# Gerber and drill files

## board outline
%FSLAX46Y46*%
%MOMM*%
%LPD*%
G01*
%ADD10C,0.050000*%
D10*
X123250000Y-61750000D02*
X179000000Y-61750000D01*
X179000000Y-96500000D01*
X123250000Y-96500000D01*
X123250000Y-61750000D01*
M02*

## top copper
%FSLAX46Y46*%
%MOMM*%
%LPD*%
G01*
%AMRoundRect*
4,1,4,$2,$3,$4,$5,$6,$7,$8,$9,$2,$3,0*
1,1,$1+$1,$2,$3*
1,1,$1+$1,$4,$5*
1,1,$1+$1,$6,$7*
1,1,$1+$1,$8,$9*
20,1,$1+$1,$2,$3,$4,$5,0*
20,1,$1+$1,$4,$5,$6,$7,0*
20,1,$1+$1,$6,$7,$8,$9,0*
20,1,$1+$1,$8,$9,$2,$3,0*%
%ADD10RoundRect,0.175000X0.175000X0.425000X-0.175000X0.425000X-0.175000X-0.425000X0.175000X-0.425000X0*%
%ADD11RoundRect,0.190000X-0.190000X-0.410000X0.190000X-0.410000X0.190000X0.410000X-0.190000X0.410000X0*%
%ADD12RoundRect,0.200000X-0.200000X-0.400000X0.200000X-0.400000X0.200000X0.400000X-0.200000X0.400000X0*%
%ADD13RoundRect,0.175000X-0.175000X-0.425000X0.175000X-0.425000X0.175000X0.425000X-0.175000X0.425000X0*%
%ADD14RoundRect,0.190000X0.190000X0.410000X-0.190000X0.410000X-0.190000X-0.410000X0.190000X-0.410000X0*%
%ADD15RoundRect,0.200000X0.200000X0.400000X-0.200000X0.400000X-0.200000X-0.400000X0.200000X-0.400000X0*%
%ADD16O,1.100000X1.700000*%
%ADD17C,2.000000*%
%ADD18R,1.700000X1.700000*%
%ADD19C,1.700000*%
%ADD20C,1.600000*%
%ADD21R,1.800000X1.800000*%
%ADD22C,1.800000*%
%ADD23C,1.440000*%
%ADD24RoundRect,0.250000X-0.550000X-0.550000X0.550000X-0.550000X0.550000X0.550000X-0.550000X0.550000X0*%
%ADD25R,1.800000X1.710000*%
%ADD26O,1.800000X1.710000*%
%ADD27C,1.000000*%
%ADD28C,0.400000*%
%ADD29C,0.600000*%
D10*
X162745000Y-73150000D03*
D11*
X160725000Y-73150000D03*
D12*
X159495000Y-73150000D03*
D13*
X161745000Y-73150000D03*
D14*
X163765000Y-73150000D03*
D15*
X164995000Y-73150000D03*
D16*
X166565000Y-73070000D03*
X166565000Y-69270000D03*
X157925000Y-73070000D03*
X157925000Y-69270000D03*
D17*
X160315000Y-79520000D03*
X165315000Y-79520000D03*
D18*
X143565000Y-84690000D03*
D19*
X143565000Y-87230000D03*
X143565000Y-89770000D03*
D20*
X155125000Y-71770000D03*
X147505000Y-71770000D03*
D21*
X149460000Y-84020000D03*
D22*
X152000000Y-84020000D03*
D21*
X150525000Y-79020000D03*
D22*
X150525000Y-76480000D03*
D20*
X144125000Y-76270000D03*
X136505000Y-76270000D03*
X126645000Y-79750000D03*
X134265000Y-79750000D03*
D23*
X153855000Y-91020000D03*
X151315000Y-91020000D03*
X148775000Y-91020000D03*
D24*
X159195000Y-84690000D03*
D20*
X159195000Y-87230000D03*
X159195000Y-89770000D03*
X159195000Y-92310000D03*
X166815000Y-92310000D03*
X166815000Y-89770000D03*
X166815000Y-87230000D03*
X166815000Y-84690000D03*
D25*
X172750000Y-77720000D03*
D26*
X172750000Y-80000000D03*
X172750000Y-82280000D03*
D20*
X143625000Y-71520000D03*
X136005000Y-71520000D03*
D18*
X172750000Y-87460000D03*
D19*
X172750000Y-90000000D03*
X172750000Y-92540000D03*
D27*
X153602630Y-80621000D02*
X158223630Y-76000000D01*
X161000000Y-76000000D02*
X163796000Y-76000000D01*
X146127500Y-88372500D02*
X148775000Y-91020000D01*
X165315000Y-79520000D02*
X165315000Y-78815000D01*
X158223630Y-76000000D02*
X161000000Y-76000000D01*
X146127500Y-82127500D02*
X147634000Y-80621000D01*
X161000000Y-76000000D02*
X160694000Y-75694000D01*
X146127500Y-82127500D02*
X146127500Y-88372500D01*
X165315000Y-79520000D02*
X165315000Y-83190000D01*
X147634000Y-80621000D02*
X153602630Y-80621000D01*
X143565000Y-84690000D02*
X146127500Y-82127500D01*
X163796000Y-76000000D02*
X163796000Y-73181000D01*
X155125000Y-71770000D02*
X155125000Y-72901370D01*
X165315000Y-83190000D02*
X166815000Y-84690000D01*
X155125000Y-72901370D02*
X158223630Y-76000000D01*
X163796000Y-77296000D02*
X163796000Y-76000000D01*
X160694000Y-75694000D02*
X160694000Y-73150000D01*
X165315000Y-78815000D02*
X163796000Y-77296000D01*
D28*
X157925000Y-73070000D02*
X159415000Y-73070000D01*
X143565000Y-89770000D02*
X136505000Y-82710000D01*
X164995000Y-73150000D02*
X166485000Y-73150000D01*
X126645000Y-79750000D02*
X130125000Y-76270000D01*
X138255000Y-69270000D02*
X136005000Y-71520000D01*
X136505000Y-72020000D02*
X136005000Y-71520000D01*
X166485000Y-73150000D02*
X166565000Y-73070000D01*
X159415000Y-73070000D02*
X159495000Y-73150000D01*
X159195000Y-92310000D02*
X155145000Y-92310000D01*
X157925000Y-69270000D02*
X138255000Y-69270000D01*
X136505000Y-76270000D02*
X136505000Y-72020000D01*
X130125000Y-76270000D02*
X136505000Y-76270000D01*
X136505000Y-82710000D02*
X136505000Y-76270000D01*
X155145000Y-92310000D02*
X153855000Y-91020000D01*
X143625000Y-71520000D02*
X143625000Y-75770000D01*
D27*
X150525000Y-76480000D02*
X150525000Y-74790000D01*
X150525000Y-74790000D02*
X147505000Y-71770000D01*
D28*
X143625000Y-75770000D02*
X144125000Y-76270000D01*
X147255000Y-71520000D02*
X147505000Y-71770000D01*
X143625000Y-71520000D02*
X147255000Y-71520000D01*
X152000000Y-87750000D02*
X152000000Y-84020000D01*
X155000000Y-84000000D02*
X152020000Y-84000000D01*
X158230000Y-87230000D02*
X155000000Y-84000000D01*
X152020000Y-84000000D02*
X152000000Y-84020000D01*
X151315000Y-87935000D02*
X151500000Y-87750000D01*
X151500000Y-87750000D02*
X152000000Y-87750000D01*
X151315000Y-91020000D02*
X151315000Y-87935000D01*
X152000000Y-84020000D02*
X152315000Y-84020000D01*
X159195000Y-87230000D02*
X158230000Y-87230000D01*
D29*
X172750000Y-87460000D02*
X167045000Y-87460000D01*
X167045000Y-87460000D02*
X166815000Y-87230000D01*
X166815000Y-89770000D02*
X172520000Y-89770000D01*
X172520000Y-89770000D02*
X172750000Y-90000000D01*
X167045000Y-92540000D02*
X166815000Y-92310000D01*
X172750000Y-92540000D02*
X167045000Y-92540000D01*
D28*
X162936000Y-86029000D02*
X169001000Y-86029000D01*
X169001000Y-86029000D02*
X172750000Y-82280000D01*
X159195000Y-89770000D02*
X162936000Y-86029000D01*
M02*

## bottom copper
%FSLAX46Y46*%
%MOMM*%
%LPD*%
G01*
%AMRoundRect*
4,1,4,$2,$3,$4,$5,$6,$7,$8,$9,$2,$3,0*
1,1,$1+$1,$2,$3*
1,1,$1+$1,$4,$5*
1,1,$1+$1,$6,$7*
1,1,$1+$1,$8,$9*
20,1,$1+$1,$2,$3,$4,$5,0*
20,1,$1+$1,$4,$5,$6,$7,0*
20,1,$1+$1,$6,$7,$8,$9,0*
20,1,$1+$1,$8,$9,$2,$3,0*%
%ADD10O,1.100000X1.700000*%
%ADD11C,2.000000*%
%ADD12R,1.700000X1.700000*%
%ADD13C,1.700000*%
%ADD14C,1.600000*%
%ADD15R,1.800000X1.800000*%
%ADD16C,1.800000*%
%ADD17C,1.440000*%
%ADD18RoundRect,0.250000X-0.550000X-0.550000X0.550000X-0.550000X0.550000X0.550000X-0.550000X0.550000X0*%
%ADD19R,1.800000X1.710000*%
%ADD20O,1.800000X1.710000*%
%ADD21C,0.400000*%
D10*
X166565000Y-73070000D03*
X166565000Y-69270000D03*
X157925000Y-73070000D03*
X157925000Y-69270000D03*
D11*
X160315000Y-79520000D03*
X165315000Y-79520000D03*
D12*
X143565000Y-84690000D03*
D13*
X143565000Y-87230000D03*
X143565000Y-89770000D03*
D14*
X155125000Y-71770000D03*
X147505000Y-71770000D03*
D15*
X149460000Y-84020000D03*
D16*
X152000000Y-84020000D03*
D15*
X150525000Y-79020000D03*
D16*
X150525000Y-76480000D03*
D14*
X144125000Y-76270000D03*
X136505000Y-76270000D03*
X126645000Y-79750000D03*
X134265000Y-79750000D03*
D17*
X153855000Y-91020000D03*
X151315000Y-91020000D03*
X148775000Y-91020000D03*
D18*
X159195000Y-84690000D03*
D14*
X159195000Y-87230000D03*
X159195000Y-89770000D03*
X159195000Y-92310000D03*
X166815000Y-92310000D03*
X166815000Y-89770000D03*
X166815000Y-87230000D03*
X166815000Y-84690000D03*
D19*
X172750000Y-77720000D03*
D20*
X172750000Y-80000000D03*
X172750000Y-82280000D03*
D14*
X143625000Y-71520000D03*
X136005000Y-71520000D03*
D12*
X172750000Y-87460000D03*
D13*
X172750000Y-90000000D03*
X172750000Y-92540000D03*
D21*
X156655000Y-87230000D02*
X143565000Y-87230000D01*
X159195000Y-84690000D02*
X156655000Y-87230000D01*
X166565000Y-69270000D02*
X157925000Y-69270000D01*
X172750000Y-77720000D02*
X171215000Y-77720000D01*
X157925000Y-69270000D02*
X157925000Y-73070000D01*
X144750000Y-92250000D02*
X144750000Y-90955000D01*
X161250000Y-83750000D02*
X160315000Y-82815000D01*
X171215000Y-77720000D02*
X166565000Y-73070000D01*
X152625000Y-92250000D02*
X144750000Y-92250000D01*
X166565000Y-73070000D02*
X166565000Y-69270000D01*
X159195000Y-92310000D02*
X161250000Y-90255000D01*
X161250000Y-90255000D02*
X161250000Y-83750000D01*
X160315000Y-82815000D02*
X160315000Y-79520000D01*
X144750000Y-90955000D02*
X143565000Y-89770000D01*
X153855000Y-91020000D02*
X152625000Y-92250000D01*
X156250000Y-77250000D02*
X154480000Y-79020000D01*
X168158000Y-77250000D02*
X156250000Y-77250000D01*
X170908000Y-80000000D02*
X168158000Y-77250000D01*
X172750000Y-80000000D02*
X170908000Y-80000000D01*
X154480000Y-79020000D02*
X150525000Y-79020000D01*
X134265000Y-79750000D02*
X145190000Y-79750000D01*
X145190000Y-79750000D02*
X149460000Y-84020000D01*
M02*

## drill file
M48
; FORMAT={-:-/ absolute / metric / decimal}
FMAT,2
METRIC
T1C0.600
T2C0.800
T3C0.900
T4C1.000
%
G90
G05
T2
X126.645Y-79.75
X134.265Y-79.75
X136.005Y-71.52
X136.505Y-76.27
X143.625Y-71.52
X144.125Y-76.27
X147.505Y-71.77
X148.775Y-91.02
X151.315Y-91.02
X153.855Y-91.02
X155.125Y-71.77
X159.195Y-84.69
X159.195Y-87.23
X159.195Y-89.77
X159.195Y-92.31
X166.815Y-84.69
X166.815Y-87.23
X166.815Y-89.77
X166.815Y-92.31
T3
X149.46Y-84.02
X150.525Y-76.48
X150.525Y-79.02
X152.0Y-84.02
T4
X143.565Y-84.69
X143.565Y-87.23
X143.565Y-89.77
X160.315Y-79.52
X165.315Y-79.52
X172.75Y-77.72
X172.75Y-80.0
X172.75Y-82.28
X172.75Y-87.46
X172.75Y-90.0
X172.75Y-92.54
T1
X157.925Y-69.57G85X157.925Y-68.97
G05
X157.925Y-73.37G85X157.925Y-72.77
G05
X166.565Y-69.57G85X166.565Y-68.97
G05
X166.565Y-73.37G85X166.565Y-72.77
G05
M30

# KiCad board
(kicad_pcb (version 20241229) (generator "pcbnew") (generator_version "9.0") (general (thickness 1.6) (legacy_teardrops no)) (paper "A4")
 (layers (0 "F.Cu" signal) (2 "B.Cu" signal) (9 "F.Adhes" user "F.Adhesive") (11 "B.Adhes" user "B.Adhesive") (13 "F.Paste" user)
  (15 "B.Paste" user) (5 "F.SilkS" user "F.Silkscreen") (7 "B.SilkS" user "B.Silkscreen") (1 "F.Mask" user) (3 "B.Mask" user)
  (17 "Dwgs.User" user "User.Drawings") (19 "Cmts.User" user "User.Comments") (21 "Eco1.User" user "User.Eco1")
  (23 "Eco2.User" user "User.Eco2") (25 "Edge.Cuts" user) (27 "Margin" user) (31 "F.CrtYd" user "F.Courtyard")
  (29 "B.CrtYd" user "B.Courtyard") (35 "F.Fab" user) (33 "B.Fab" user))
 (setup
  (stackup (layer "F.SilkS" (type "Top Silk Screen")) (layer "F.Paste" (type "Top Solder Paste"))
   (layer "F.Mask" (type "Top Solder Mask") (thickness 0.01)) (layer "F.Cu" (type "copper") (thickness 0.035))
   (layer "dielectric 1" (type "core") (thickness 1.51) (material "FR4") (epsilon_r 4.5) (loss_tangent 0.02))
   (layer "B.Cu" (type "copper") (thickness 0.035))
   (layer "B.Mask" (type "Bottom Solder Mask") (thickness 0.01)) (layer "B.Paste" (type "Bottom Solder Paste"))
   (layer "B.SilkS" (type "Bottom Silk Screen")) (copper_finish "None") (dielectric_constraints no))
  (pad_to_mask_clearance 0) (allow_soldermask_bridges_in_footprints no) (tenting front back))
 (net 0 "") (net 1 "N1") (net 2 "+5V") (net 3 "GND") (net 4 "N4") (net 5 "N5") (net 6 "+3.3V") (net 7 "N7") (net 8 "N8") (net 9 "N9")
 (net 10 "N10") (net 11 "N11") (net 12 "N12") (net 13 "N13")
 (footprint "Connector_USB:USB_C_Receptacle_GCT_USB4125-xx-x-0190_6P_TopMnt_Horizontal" (layer "F.Cu") (at 162.245 70.07 180)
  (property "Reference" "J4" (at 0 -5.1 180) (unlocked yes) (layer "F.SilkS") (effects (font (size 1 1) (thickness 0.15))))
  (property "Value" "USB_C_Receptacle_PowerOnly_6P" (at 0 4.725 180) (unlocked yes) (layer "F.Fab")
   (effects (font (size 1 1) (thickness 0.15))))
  (pad "A5" smd roundrect (at -0.5 -3.08 180) (size 0.7 1.2) (layers "F.Cu" "F.Mask" "F.Paste") (roundrect_rratio 0.25) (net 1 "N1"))
  (pad "A9" smd roundrect (at 1.52 -3.08) (size 0.76 1.2) (layers "F.Cu" "F.Mask" "F.Paste") (roundrect_rratio 0.25) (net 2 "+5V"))
  (pad "A12" smd roundrect (at 2.75 -3.08) (size 0.8 1.2) (layers "F.Cu" "F.Mask" "F.Paste") (roundrect_rratio 0.25) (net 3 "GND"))
  (pad "B5" smd roundrect (at 0.5 -3.08) (size 0.7 1.2) (layers "F.Cu" "F.Mask" "F.Paste") (roundrect_rratio 0.25) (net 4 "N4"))
  (pad "B9" smd roundrect (at -1.52 -3.08 180) (size 0.76 1.2) (layers "F.Cu" "F.Mask" "F.Paste") (roundrect_rratio 0.25) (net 2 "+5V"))
  (pad "B12" smd roundrect (at -2.75 -3.08 180) (size 0.8 1.2) (layers "F.Cu" "F.Mask" "F.Paste") (roundrect_rratio 0.25) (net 3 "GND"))
  (pad "S1" thru_hole oval (at -4.32 -3 180) (size 1.1 1.7) (drill oval 0.6 1.2) (layers "*.Cu" "*.Mask" "F.Paste")
   (remove_unused_layers no) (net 3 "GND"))
  (pad "S1" thru_hole oval (at -4.32 0.8 180) (size 1.1 1.7) (drill oval 0.6 1.2) (layers "*.Cu" "*.Mask" "F.Paste")
   (remove_unused_layers no) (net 3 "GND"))
  (pad "S1" thru_hole oval (at 4.32 -3 180) (size 1.1 1.7) (drill oval 0.6 1.2) (layers "*.Cu" "*.Mask" "F.Paste") (remove_unused_layers no)
   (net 3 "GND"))
  (pad "S1" thru_hole oval (at 4.32 0.8 180) (size 1.1 1.7) (drill oval 0.6 1.2) (layers "*.Cu" "*.Mask" "F.Paste")
   (remove_unused_layers no) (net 3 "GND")))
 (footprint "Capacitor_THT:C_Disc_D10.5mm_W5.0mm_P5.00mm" (layer "F.Cu") (at 160.315 79.52)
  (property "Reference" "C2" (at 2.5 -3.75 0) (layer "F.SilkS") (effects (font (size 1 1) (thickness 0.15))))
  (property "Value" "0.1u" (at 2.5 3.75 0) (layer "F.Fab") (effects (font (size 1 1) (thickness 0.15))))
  (pad "1" thru_hole circle (at 0 0) (size 2 2) (drill 1) (layers "*.Cu" "*.Mask") (remove_unused_layers no) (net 3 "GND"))
  (pad "2" thru_hole circle (at 5 0) (size 2 2) (drill 1) (layers "*.Cu" "*.Mask") (remove_unused_layers no) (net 2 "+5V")))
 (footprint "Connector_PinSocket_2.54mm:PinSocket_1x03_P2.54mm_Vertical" (layer "F.Cu") (at 143.565 84.69)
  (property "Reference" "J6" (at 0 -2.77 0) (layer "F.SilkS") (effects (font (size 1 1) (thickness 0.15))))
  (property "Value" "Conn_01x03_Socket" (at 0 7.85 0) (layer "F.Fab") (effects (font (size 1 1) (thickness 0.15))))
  (pad "1" thru_hole rect (at 0 0) (size 1.7 1.7) (drill 1) (layers "*.Cu" "*.Mask") (remove_unused_layers no) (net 2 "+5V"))
  (pad "2" thru_hole circle (at 0 2.54) (size 1.7 1.7) (drill 1) (layers "*.Cu" "*.Mask") (remove_unused_layers no) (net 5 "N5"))
  (pad "3" thru_hole circle (at 0 5.08) (size 1.7 1.7) (drill 1) (layers "*.Cu" "*.Mask") (remove_unused_layers no) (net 3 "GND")))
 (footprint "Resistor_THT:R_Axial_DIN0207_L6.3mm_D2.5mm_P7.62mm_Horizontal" (layer "F.Cu") (at 155.125 71.77 180)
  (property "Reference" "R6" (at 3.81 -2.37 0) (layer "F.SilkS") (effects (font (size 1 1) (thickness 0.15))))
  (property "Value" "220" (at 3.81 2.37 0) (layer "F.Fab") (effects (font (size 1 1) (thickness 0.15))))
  (pad "1" thru_hole circle (at 0 0 180) (size 1.6 1.6) (drill 0.8) (layers "*.Cu" "*.Mask") (remove_unused_layers no) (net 2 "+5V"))
  (pad "2" thru_hole circle (at 7.62 0 180) (size 1.6 1.6) (drill 0.8) (layers "*.Cu" "*.Mask") (remove_unused_layers no) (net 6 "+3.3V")))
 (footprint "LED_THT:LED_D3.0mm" (layer "F.Cu") (at 149.46 84.02)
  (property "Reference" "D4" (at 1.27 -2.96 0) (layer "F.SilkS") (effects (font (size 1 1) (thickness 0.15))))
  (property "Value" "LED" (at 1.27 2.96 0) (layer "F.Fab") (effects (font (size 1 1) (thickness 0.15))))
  (pad "1" thru_hole rect (at 0 0) (size 1.8 1.8) (drill 0.9) (layers "*.Cu" "*.Mask") (remove_unused_layers no) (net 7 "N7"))
  (pad "2" thru_hole circle (at 2.54 0) (size 1.8 1.8) (drill 0.9) (layers "*.Cu" "*.Mask") (remove_unused_layers no) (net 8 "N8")))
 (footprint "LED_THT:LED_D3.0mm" (layer "F.Cu") (at 150.525 79.02 90)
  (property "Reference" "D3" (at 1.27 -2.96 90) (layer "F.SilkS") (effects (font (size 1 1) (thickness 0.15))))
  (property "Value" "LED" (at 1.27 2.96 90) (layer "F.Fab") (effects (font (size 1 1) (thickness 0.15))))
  (pad "1" thru_hole rect (at 0 0 90) (size 1.8 1.8) (drill 0.9) (layers "*.Cu" "*.Mask") (remove_unused_layers no) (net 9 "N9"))
  (pad "2" thru_hole circle (at 2.54 0 90) (size 1.8 1.8) (drill 0.9) (layers "*.Cu" "*.Mask") (remove_unused_layers no) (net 6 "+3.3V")))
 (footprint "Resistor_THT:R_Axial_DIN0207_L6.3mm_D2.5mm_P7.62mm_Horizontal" (layer "F.Cu") (at 144.125 76.27 180)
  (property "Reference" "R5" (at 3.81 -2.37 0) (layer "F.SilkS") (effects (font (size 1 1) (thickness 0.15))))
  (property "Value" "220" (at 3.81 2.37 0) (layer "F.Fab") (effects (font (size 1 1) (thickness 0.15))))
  (pad "1" thru_hole circle (at 0 0 180) (size 1.6 1.6) (drill 0.8) (layers "*.Cu" "*.Mask") (remove_unused_layers no) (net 6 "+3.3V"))
  (pad "2" thru_hole circle (at 7.62 0 180) (size 1.6 1.6) (drill 0.8) (layers "*.Cu" "*.Mask") (remove_unused_layers no) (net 3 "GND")))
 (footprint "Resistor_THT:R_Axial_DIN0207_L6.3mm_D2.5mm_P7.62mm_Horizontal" (layer "F.Cu") (at 126.645 79.75)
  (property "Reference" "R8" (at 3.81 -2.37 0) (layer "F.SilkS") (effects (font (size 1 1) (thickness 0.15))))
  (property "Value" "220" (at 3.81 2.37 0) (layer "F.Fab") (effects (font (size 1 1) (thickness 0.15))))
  (pad "1" thru_hole circle (at 0 0) (size 1.6 1.6) (drill 0.8) (layers "*.Cu" "*.Mask") (remove_unused_layers no) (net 3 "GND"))
  (pad "2" thru_hole circle (at 7.62 0) (size 1.6 1.6) (drill 0.8) (layers "*.Cu" "*.Mask") (remove_unused_layers no) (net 7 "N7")))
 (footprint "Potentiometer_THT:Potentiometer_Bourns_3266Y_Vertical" (layer "F.Cu") (at 153.855 91.02)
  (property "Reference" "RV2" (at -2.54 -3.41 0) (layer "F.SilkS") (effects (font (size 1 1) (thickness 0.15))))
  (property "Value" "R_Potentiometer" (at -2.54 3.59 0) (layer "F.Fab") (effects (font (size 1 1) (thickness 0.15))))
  (pad "1" thru_hole circle (at 0 0) (size 1.44 1.44) (drill 0.8) (layers "*.Cu" "*.Mask") (remove_unused_layers no) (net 3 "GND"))
  (pad "2" thru_hole circle (at -2.54 0) (size 1.44 1.44) (drill 0.8) (layers "*.Cu" "*.Mask") (remove_unused_layers no) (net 8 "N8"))
  (pad "3" thru_hole circle (at -5.08 0) (size 1.44 1.44) (drill 0.8) (layers "*.Cu" "*.Mask") (remove_unused_layers no) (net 2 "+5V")))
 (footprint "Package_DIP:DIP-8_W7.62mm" (layer "F.Cu") (at 159.195 84.69)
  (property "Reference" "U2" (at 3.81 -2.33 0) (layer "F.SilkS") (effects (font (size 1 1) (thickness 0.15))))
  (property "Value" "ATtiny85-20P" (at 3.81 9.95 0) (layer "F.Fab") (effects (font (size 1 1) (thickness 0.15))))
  (pad "1" thru_hole roundrect (at 0 0) (size 1.6 1.6) (drill 0.8) (layers "*.Cu" "*.Mask") (remove_unused_layers no)
   (roundrect_rratio 0.15625) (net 5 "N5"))
  (pad "2" thru_hole circle (at 0 2.54) (size 1.6 1.6) (drill 0.8) (layers "*.Cu" "*.Mask") (remove_unused_layers no) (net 8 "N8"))
  (pad "3" thru_hole circle (at 0 5.08) (size 1.6 1.6) (drill 0.8) (layers "*.Cu" "*.Mask") (remove_unused_layers no) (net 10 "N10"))
  (pad "4" thru_hole circle (at 0 7.62) (size 1.6 1.6) (drill 0.8) (layers "*.Cu" "*.Mask") (remove_unused_layers no) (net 3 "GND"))
  (pad "5" thru_hole circle (at 7.62 7.62) (size 1.6 1.6) (drill 0.8) (layers "*.Cu" "*.Mask") (remove_unused_layers no) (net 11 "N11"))
  (pad "6" thru_hole circle (at 7.62 5.08) (size 1.6 1.6) (drill 0.8) (layers "*.Cu" "*.Mask") (remove_unused_layers no) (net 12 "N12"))
  (pad "7" thru_hole circle (at 7.62 2.54) (size 1.6 1.6) (drill 0.8) (layers "*.Cu" "*.Mask") (remove_unused_layers no) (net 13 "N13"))
  (pad "8" thru_hole circle (at 7.62 0) (size 1.6 1.6) (drill 0.8) (layers "*.Cu" "*.Mask") (remove_unused_layers no) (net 2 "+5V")))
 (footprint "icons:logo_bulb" (layer "F.Cu") (at 128.5 91.5)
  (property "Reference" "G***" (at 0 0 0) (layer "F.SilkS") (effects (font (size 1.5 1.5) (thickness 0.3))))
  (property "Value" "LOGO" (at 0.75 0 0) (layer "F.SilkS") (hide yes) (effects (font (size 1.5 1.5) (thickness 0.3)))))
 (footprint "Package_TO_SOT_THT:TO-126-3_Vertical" (layer "F.Cu") (at 172.75 77.72 -90)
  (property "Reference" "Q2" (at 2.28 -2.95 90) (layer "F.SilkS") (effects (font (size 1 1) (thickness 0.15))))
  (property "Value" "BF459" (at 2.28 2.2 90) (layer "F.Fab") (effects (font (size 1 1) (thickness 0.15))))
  (pad "1" thru_hole rect (at 0 0 270) (size 1.71 1.8) (drill 1) (layers "*.Cu" "*.Mask") (remove_unused_layers no) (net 3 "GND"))
  (pad "2" thru_hole oval (at 2.28 0 270) (size 1.71 1.8) (drill 1) (layers "*.Cu" "*.Mask") (remove_unused_layers no) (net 9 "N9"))
  (pad "3" thru_hole oval (at 4.56 0 270) (size 1.71 1.8) (drill 1) (layers "*.Cu" "*.Mask") (remove_unused_layers no) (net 10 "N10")))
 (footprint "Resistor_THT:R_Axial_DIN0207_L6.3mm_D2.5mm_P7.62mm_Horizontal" (layer "F.Cu") (at 143.625 71.52 180)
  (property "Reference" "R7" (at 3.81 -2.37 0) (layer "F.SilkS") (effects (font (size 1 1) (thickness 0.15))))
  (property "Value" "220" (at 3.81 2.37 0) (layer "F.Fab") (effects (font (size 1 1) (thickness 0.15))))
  (pad "1" thru_hole circle (at 0 0 180) (size 1.6 1.6) (drill 0.8) (layers "*.Cu" "*.Mask") (remove_unused_layers no) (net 6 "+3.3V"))
  (pad "2" thru_hole circle (at 7.62 0 180) (size 1.6 1.6) (drill 0.8) (layers "*.Cu" "*.Mask") (remove_unused_layers no) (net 3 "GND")))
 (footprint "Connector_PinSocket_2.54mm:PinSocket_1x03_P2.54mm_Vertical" (layer "F.Cu") (at 172.75 87.46)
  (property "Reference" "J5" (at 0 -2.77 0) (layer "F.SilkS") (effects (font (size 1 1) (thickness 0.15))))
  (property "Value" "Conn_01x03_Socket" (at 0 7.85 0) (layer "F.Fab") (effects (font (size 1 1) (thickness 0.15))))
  (pad "1" thru_hole rect (at 0 0) (size 1.7 1.7) (drill 1) (layers "*.Cu" "*.Mask") (remove_unused_layers no) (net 13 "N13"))
  (pad "2" thru_hole circle (at 0 2.54) (size 1.7 1.7) (drill 1) (layers "*.Cu" "*.Mask") (remove_unused_layers no) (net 12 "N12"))
  (pad "3" thru_hole circle (at 0 5.08) (size 1.7 1.7) (drill 1) (layers "*.Cu" "*.Mask") (remove_unused_layers no) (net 11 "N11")))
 (gr_rect (start 123.25 61.75) (end 179 96.5) (stroke (width 0.05) (type default)) (fill no) (layer "Edge.Cuts"))
 (segment (start 153.60263 80.621) (end 158.22363 76) (width 1) (layer "F.Cu") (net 2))
 (segment (start 161 76) (end 163.796 76) (width 1) (layer "F.Cu") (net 2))
 (segment (start 146.1275 88.3725) (end 148.775 91.02) (width 1) (layer "F.Cu") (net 2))
 (segment (start 165.315 79.52) (end 165.315 78.815) (width 1) (layer "F.Cu") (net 2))
 (segment (start 158.22363 76) (end 161 76) (width 1) (layer "F.Cu") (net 2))
 (segment (start 146.1275 82.1275) (end 147.634 80.621) (width 1) (layer "F.Cu") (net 2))
 (segment (start 161 76) (end 160.694 75.694) (width 1) (layer "F.Cu") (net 2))
 (segment (start 146.1275 82.1275) (end 146.1275 88.3725) (width 1) (layer "F.Cu") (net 2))
 (segment (start 165.315 79.52) (end 165.315 83.19) (width 1) (layer "F.Cu") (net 2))
 (segment (start 147.634 80.621) (end 153.60263 80.621) (width 1) (layer "F.Cu") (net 2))
 (segment (start 143.565 84.69) (end 146.1275 82.1275) (width 1) (layer "F.Cu") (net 2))
 (segment (start 163.796 76) (end 163.796 73.181) (width 1) (layer "F.Cu") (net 2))
 (segment (start 155.125 71.77) (end 155.125 72.90137) (width 1) (layer "F.Cu") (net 2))
 (segment (start 165.315 83.19) (end 166.815 84.69) (width 1) (layer "F.Cu") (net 2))
 (segment (start 155.125 72.90137) (end 158.22363 76) (width 1) (layer "F.Cu") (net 2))
 (segment (start 163.796 77.296) (end 163.796 76) (width 1) (layer "F.Cu") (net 2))
 (segment (start 160.694 75.694) (end 160.694 73.15) (width 1) (layer "F.Cu") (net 2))
 (segment (start 165.315 78.815) (end 163.796 77.296) (width 1) (layer "F.Cu") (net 2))
 (segment (start 156.655 87.23) (end 143.565 87.23) (width 0.4) (layer "B.Cu") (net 5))
 (segment (start 159.195 84.69) (end 156.655 87.23) (width 0.4) (layer "B.Cu") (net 5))
 (segment (start 157.925 73.07) (end 159.415 73.07) (width 0.4) (layer "F.Cu") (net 3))
 (segment (start 143.565 89.77) (end 136.505 82.71) (width 0.4) (layer "F.Cu") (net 3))
 (segment (start 164.995 73.15) (end 166.485 73.15) (width 0.4) (layer "F.Cu") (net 3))
 (segment (start 126.645 79.75) (end 130.125 76.27) (width 0.4) (layer "F.Cu") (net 3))
 (segment (start 138.255 69.27) (end 136.005 71.52) (width 0.4) (layer "F.Cu") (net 3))
 (segment (start 136.505 72.02) (end 136.005 71.52) (width 0.4) (layer "F.Cu") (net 3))
 (segment (start 166.485 73.15) (end 166.565 73.07) (width 0.4) (layer "F.Cu") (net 3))
 (segment (start 159.415 73.07) (end 159.495 73.15) (width 0.4) (layer "F.Cu") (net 3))
 (segment (start 159.195 92.31) (end 155.145 92.31) (width 0.4) (layer "F.Cu") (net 3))
 (segment (start 157.925 69.27) (end 138.255 69.27) (width 0.4) (layer "F.Cu") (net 3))
 (segment (start 136.505 76.27) (end 136.505 72.02) (width 0.4) (layer "F.Cu") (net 3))
 (segment (start 130.125 76.27) (end 136.505 76.27) (width 0.4) (layer "F.Cu") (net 3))
 (segment (start 136.505 82.71) (end 136.505 76.27) (width 0.4) (layer "F.Cu") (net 3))
 (segment (start 155.145 92.31) (end 153.855 91.02) (width 0.4) (layer "F.Cu") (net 3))
 (segment (start 166.565 69.27) (end 157.925 69.27) (width 0.4) (layer "B.Cu") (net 3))
 (segment (start 172.75 77.72) (end 171.215 77.72) (width 0.4) (layer "B.Cu") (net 3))
 (segment (start 157.925 69.27) (end 157.925 73.07) (width 0.4) (layer "B.Cu") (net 3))
 (segment (start 144.75 92.25) (end 144.75 90.955) (width 0.4) (layer "B.Cu") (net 3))
 (segment (start 161.25 83.75) (end 160.315 82.815) (width 0.4) (layer "B.Cu") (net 3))
 (segment (start 171.215 77.72) (end 166.565 73.07) (width 0.4) (layer "B.Cu") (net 3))
 (segment (start 152.625 92.25) (end 144.75 92.25) (width 0.4) (layer "B.Cu") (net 3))
 (segment (start 166.565 73.07) (end 166.565 69.27) (width 0.4) (layer "B.Cu") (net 3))
 (segment (start 159.195 92.31) (end 161.25 90.255) (width 0.4) (layer "B.Cu") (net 3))
 (segment (start 161.25 90.255) (end 161.25 83.75) (width 0.4) (layer "B.Cu") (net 3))
 (segment (start 160.315 82.815) (end 160.315 79.52) (width 0.4) (layer "B.Cu") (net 3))
 (segment (start 144.75 90.955) (end 143.565 89.77) (width 0.4) (layer "B.Cu") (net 3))
 (segment (start 153.855 91.02) (end 152.625 92.25) (width 0.4) (layer "B.Cu") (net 3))
 (segment (start 156.25 77.25) (end 154.48 79.02) (width 0.4) (layer "B.Cu") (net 9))
 (segment (start 168.158 77.25) (end 156.25 77.25) (width 0.4) (layer "B.Cu") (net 9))
 (segment (start 170.908 80) (end 168.158 77.25) (width 0.4) (layer "B.Cu") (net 9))
 (segment (start 172.75 80) (end 170.908 80) (width 0.4) (layer "B.Cu") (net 9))
 (segment (start 154.48 79.02) (end 150.525 79.02) (width 0.4) (layer "B.Cu") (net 9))
 (segment (start 143.625 71.52) (end 143.625 75.77) (width 0.4) (layer "F.Cu") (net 6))
 (segment (start 150.525 76.48) (end 150.525 74.79) (width 1) (layer "F.Cu") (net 6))
 (segment (start 150.525 74.79) (end 147.505 71.77) (width 1) (layer "F.Cu") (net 6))
 (segment (start 143.625 75.77) (end 144.125 76.27) (width 0.4) (layer "F.Cu") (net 6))
 (segment (start 147.255 71.52) (end 147.505 71.77) (width 0.4) (layer "F.Cu") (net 6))
 (segment (start 143.625 71.52) (end 147.255 71.52) (width 0.4) (layer "F.Cu") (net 6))
 (segment (start 134.265 79.75) (end 145.19 79.75) (width 0.4) (layer "B.Cu") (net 7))
 (segment (start 145.19 79.75) (end 149.46 84.02) (width 0.4) (layer "B.Cu") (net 7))
 (segment (start 152 87.75) (end 152 84.02) (width 0.4) (layer "F.Cu") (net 8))
 (segment (start 155 84) (end 152.02 84) (width 0.4) (layer "F.Cu") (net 8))
 (segment (start 158.23 87.23) (end 155 84) (width 0.4) (layer "F.Cu") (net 8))
 (segment (start 152.02 84) (end 152 84.02) (width 0.4) (layer "F.Cu") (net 8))
 (segment (start 151.315 87.935) (end 151.5 87.75) (width 0.4) (layer "F.Cu") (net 8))
 (segment (start 151.5 87.75) (end 152 87.75) (width 0.4) (layer "F.Cu") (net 8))
 (segment (start 151.315 91.02) (end 151.315 87.935) (width 0.4) (layer "F.Cu") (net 8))
 (segment (start 152 84.02) (end 152.315 84.02) (width 0.4) (layer "F.Cu") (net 8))
 (segment (start 159.195 87.23) (end 158.23 87.23) (width 0.4) (layer "F.Cu") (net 8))
 (segment (start 172.75 87.46) (end 167.045 87.46) (width 0.6) (layer "F.Cu") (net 13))
 (segment (start 167.045 87.46) (end 166.815 87.23) (width 0.6) (layer "F.Cu") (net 13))
 (segment (start 166.815 89.77) (end 172.52 89.77) (width 0.6) (layer "F.Cu") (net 12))
 (segment (start 172.52 89.77) (end 172.75 90) (width 0.6) (layer "F.Cu") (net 12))
 (segment (start 167.045 92.54) (end 166.815 92.31) (width 0.6) (layer "F.Cu") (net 11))
 (segment (start 172.75 92.54) (end 167.045 92.54) (width 0.6) (layer "F.Cu") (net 11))
 (segment (start 162.936 86.029) (end 169.001 86.029) (width 0.4) (layer "F.Cu") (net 10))
 (segment (start 169.001 86.029) (end 172.75 82.28) (width 0.4) (layer "F.Cu") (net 10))
 (segment (start 159.195 89.77) (end 162.936 86.029) (width 0.4) (layer "F.Cu") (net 10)))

